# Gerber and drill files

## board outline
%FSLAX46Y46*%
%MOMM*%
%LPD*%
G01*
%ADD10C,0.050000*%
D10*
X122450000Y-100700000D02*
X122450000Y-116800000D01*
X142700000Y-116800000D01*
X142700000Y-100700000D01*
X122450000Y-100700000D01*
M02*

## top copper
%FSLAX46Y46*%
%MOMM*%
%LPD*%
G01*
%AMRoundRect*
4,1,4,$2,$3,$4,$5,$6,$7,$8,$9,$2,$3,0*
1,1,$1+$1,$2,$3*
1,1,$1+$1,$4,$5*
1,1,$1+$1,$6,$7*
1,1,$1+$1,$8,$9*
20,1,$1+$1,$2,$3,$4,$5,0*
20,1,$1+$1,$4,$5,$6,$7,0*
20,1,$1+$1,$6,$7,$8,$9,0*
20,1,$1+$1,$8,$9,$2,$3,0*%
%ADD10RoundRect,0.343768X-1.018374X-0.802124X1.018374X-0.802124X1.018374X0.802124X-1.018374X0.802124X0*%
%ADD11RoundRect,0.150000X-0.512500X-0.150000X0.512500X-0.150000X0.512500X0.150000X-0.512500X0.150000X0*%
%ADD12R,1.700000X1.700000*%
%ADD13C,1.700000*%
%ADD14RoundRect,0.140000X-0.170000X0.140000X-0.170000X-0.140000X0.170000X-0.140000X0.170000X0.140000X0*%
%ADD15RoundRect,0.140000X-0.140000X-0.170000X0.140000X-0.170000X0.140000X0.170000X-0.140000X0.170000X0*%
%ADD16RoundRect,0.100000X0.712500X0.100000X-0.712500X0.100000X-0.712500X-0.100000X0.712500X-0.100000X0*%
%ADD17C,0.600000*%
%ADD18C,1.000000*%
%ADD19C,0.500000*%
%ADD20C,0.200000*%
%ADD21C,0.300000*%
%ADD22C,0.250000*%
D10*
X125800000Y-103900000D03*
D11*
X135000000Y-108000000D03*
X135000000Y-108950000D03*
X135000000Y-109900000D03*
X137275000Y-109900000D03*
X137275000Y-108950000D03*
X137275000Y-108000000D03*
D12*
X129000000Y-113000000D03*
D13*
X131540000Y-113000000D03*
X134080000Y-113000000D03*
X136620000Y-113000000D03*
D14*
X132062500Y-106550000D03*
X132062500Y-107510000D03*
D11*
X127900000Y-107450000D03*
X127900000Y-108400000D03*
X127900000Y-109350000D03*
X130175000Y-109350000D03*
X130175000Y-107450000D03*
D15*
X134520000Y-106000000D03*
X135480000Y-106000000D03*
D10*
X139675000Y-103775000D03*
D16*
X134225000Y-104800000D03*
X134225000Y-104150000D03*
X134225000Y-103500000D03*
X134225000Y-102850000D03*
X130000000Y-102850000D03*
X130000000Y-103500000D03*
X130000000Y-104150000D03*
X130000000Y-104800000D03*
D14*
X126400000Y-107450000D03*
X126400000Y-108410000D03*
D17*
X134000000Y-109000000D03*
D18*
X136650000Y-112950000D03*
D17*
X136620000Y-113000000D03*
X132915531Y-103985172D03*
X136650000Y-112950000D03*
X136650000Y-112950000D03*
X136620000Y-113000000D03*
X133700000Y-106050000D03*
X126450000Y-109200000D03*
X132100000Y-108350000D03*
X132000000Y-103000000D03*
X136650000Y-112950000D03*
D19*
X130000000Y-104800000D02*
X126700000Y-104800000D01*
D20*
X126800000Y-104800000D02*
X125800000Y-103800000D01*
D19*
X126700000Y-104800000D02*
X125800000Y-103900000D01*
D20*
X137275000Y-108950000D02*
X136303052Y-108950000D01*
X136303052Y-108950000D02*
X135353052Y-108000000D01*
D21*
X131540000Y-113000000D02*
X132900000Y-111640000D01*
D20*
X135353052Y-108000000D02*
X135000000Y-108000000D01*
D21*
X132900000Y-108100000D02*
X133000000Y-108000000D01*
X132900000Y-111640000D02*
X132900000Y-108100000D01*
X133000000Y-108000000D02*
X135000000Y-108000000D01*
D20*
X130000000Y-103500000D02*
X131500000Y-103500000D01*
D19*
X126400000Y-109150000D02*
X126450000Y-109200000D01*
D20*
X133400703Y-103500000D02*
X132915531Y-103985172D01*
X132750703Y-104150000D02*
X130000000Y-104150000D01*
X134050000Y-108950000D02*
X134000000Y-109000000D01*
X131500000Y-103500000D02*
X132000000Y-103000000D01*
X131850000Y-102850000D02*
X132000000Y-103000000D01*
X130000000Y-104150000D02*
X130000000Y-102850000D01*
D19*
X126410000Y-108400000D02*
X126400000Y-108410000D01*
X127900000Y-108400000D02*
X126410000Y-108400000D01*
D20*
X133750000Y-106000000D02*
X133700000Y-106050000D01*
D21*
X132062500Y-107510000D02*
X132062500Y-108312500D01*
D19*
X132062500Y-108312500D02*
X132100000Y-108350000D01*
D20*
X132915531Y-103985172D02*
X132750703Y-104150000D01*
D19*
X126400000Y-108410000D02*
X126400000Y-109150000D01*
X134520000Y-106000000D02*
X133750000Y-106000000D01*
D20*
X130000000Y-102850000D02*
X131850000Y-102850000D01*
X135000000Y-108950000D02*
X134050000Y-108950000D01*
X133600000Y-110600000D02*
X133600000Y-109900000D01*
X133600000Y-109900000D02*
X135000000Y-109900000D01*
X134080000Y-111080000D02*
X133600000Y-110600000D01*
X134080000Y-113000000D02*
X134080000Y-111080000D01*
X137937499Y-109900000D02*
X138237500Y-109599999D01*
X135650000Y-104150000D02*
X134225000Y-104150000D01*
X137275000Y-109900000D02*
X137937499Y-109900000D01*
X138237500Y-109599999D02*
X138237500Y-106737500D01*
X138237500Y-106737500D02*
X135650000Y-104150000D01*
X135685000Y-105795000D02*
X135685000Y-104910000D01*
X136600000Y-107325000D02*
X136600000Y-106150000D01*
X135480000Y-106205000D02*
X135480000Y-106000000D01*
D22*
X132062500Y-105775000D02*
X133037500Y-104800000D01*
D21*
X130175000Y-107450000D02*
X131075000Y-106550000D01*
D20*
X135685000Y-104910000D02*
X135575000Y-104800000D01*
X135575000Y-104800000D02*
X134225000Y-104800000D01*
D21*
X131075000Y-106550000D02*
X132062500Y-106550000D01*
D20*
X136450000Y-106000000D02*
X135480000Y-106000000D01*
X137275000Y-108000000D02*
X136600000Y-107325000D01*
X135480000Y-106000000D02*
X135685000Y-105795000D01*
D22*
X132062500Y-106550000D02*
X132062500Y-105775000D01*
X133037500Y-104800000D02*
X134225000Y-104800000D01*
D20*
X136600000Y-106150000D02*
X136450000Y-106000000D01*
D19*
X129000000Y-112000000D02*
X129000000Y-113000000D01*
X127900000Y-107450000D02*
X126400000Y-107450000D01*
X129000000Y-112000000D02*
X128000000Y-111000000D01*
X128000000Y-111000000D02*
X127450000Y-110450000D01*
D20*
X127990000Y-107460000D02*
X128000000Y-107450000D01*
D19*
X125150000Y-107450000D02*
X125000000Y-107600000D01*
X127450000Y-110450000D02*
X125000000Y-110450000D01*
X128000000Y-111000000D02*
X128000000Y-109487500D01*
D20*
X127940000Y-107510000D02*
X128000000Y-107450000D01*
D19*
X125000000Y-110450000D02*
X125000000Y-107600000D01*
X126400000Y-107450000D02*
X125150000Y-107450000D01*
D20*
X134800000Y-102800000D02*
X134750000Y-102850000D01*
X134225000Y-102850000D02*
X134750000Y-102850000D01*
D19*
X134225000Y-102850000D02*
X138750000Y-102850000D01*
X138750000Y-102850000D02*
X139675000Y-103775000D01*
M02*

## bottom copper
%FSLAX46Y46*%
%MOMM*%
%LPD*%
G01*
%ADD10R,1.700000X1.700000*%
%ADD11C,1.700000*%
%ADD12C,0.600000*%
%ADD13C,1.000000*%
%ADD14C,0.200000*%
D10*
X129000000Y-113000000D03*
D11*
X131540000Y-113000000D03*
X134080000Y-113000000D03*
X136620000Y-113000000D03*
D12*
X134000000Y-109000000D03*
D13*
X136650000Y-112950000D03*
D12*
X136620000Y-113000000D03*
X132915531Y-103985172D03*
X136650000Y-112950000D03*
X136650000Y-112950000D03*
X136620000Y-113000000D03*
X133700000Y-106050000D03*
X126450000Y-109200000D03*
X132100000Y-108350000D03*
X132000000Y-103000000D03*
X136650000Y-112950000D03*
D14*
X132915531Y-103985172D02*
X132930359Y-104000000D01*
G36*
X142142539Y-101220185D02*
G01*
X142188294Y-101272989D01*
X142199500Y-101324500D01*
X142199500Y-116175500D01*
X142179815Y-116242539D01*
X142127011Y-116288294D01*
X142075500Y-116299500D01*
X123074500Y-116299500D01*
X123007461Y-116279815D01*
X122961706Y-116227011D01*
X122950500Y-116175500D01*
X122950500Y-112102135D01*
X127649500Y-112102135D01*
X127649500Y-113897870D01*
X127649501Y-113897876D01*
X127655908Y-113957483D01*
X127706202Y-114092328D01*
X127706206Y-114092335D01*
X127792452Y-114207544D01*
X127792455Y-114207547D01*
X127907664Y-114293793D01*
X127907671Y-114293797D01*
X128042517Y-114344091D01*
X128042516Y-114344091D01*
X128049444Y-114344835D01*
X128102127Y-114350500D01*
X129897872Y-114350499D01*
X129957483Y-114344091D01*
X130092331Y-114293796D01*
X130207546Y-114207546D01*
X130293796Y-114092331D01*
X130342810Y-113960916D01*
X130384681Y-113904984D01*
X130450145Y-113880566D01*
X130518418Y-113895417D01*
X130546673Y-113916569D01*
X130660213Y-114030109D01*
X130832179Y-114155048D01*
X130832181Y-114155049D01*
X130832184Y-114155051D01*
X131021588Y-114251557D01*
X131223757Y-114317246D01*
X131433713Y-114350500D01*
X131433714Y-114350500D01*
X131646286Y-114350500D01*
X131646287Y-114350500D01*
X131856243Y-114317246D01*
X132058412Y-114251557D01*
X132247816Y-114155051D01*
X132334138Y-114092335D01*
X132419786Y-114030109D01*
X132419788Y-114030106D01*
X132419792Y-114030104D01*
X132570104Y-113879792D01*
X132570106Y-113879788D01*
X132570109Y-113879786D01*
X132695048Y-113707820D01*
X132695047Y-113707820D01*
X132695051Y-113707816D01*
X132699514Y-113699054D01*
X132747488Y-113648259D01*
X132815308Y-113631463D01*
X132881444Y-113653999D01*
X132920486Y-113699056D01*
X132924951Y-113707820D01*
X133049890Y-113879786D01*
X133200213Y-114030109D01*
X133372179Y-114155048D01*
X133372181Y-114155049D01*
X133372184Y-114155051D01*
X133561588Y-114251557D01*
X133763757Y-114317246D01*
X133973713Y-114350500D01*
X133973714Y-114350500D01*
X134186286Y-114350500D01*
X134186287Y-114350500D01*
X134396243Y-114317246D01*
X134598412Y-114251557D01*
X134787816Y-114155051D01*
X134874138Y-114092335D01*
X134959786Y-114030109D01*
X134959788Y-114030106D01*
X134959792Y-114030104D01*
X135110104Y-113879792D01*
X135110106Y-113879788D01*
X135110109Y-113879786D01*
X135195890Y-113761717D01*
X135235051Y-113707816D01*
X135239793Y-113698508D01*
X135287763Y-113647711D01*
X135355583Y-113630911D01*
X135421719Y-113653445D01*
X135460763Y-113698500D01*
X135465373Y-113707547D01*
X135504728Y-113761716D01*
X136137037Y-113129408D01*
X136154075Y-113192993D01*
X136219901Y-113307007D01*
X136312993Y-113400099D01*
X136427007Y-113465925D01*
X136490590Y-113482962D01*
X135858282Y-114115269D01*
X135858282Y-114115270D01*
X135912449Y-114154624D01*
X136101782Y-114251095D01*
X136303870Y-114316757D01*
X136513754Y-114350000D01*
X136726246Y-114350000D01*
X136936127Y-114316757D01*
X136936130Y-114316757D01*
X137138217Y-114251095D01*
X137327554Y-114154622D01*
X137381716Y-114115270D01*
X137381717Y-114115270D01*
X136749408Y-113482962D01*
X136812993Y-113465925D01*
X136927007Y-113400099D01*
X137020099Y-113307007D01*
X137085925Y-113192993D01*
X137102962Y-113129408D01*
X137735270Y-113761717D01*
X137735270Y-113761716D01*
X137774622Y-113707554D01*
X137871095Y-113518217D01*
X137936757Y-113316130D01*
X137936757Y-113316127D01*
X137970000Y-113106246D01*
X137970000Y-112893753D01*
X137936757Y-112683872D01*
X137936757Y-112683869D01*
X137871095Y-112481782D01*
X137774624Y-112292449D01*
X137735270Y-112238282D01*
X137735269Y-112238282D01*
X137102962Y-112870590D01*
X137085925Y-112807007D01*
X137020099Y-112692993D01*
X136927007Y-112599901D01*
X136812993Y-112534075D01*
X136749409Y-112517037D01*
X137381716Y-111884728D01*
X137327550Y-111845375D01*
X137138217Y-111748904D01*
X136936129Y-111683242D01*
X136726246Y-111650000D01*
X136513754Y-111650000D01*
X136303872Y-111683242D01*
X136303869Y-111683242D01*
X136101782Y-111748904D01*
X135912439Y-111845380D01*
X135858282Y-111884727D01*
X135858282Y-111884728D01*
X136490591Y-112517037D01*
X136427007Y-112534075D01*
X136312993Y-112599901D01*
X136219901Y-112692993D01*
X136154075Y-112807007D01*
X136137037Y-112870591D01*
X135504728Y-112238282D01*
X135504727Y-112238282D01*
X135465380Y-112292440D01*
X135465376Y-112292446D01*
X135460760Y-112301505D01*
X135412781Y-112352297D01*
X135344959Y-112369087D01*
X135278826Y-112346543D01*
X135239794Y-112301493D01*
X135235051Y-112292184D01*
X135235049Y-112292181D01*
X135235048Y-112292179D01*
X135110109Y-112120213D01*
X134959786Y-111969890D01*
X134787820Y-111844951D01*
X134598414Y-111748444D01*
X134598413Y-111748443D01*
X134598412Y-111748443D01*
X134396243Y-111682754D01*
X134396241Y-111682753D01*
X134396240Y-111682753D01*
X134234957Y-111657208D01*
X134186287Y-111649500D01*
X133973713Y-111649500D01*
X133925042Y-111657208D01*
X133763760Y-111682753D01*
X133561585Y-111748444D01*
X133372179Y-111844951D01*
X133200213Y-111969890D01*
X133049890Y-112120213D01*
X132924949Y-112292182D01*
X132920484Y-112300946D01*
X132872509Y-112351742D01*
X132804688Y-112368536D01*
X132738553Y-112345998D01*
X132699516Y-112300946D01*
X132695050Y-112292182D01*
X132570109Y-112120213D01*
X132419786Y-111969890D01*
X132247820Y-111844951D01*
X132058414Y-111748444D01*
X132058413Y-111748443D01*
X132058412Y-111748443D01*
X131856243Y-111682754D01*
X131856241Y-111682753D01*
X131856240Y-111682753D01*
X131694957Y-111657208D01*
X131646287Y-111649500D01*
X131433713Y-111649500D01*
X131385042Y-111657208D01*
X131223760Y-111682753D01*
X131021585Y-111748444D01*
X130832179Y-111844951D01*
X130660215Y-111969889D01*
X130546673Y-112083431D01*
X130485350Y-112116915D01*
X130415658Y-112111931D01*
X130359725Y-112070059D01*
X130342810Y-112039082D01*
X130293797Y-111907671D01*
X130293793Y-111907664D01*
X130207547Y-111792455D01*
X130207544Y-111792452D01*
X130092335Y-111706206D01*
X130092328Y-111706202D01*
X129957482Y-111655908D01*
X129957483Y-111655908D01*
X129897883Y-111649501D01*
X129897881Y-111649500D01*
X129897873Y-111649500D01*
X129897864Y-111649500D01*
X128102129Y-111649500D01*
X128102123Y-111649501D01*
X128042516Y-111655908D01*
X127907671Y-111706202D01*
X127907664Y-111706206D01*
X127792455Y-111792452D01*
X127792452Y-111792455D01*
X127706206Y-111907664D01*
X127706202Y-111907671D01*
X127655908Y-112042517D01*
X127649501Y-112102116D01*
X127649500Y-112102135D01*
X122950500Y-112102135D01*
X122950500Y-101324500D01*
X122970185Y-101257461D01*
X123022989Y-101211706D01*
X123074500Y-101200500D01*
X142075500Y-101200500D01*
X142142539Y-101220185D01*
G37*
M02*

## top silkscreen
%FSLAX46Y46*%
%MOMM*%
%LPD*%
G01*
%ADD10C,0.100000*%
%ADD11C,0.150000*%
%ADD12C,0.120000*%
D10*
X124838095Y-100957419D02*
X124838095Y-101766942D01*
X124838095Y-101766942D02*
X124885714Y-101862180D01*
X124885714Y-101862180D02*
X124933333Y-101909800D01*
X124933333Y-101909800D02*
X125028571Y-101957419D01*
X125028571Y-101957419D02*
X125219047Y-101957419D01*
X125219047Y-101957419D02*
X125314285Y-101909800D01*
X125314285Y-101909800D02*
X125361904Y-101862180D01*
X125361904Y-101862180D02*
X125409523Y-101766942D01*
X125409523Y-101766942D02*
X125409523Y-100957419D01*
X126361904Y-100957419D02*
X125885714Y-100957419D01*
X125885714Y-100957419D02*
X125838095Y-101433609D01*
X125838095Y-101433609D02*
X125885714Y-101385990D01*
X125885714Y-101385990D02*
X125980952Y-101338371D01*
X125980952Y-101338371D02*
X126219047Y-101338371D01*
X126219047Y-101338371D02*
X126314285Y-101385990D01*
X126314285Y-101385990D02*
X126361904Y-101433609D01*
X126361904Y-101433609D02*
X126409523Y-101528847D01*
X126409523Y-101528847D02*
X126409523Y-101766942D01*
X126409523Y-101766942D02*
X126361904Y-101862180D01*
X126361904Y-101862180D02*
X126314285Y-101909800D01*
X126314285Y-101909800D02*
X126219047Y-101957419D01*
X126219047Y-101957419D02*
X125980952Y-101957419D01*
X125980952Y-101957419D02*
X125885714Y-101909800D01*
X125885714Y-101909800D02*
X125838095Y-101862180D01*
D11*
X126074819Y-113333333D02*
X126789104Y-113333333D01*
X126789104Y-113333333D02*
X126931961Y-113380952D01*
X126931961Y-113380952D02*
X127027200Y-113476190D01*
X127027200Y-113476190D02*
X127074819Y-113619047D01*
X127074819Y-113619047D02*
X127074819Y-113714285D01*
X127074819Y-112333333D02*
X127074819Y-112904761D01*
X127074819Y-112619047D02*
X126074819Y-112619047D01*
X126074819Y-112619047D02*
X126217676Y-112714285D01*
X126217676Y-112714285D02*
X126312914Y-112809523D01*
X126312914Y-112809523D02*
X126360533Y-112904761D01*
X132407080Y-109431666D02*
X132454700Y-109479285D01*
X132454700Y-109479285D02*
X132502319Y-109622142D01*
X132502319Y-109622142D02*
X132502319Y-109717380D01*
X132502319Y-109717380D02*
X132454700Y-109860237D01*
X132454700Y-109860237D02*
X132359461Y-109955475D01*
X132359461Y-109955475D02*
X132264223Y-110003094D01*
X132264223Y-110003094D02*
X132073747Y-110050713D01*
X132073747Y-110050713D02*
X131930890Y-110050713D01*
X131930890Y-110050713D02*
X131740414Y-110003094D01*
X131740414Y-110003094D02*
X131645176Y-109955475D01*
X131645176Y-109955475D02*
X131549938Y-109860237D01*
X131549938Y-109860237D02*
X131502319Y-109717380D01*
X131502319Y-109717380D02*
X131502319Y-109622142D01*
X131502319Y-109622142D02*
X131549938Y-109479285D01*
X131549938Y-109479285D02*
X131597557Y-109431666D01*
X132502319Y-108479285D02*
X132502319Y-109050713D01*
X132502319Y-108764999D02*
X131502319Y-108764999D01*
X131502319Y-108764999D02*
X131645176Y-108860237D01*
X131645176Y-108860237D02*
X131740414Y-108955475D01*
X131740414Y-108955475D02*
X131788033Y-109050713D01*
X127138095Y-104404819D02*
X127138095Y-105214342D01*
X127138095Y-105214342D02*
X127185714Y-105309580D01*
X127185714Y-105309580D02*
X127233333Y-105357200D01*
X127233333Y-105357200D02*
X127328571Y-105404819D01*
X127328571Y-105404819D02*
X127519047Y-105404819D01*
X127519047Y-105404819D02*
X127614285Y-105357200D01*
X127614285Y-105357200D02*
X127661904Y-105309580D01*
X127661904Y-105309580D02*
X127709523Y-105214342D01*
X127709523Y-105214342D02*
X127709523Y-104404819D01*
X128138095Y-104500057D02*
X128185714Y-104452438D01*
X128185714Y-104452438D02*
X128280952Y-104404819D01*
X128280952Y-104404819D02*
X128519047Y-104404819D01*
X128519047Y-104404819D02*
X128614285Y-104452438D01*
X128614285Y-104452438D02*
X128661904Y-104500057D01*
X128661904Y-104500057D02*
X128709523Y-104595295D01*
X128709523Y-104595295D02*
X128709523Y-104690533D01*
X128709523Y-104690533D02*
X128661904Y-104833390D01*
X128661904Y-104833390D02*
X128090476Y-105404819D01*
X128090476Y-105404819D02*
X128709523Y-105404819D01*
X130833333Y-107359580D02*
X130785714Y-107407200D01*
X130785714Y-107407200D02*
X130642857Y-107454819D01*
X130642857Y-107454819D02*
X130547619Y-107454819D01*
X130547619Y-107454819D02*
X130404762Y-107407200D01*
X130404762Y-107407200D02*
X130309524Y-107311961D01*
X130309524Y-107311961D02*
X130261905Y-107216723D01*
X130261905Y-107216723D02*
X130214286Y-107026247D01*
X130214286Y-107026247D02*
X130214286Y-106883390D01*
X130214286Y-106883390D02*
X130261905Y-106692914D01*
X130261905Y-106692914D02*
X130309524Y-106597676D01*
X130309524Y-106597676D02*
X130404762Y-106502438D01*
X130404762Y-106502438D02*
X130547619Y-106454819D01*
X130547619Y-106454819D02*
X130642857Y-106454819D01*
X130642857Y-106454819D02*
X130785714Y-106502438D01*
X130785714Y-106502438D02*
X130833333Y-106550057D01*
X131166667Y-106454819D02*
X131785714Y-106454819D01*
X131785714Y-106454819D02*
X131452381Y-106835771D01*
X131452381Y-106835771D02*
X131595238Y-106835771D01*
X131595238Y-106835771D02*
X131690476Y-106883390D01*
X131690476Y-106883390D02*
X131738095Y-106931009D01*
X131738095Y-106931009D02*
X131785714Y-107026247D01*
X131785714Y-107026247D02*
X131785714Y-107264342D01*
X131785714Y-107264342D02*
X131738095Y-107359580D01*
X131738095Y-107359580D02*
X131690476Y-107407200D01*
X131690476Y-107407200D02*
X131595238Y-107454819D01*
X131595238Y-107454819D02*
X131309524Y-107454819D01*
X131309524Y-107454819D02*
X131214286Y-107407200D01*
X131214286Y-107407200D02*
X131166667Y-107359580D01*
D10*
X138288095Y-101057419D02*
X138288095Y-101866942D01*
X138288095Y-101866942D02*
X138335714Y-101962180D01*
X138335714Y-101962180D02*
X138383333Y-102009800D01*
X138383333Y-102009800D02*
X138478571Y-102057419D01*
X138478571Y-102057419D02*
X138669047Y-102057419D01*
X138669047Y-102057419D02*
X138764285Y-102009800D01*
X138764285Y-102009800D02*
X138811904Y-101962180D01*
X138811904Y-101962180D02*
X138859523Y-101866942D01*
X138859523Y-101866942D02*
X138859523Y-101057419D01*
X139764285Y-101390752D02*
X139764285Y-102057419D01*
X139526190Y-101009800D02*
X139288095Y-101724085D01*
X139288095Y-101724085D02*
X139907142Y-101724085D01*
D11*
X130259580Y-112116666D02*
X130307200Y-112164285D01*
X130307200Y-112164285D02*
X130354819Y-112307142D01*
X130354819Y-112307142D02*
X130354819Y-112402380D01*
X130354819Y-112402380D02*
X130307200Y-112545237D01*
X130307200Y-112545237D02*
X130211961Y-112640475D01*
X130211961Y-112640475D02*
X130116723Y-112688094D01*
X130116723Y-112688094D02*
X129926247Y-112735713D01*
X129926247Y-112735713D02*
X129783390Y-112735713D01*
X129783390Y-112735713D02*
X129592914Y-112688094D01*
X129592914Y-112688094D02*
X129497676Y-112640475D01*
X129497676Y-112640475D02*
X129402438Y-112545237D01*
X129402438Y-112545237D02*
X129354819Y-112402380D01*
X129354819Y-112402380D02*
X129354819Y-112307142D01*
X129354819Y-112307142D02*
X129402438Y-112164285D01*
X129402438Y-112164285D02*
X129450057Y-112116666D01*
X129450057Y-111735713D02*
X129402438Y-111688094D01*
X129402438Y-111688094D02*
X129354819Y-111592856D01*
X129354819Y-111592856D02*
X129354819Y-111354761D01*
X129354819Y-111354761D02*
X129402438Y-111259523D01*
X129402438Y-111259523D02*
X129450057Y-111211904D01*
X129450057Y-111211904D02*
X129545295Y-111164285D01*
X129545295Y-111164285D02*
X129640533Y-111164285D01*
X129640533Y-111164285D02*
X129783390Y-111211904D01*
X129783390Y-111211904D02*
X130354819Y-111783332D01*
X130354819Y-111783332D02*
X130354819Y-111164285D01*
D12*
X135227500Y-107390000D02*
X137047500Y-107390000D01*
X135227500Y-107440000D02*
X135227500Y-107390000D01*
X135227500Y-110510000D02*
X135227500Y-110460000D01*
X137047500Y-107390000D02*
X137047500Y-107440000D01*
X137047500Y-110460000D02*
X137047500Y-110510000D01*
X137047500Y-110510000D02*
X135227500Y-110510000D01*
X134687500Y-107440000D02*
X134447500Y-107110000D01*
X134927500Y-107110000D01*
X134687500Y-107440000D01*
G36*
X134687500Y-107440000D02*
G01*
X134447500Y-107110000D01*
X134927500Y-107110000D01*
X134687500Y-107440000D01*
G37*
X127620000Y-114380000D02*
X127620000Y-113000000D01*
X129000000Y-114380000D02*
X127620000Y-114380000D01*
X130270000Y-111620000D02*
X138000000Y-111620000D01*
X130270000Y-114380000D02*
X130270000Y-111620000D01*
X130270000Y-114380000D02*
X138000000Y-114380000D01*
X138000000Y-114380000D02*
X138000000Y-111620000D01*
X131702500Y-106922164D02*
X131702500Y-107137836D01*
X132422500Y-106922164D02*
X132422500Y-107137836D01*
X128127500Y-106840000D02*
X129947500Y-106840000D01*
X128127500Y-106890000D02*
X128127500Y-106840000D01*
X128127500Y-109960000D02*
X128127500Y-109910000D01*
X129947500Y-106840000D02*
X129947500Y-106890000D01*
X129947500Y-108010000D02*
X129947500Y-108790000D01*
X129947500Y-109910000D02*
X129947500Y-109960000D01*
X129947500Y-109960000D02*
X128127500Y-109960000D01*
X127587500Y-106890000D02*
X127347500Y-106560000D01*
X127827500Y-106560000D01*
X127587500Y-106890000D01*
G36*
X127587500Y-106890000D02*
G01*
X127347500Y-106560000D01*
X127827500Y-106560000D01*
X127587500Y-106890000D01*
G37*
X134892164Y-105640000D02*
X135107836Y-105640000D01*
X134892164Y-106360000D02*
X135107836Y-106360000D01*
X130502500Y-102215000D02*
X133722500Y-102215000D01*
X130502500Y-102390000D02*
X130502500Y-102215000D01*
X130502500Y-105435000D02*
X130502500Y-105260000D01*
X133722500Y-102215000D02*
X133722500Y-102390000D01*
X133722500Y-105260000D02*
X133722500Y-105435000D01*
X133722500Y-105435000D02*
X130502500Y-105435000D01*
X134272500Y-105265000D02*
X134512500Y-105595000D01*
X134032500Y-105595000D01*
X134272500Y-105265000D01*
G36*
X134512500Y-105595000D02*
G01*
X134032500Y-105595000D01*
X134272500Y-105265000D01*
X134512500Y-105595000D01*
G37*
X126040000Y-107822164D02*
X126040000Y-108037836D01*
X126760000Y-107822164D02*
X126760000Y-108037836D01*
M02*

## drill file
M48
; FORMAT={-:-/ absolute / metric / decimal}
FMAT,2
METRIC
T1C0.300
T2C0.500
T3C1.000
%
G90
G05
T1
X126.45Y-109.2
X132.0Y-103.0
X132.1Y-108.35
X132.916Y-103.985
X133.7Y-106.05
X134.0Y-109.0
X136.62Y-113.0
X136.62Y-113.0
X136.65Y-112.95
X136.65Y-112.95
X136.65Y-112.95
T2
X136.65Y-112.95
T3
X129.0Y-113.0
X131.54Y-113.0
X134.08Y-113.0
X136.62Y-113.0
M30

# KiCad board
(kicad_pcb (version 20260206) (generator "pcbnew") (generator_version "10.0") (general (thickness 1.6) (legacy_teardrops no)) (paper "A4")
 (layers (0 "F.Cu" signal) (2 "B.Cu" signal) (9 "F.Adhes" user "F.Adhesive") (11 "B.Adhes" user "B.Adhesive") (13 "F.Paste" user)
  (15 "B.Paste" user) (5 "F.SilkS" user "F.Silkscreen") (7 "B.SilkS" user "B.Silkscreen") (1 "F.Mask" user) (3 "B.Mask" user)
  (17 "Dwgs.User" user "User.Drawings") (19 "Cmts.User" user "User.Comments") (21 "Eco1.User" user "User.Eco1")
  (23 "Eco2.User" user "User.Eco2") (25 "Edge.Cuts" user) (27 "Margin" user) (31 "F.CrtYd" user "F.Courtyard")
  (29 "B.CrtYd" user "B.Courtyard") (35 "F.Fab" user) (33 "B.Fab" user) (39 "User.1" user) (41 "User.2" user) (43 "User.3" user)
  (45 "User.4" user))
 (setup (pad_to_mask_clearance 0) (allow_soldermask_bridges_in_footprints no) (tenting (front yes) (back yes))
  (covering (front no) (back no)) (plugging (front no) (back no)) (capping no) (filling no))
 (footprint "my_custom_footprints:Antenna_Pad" (layer "F.Cu") (at 125.8 103.9)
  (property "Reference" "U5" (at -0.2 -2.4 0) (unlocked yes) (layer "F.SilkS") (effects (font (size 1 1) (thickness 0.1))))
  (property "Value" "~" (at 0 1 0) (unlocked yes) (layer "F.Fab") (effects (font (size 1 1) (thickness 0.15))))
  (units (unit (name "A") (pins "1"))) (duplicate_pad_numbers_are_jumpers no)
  (pad "1" smd roundrect (at 0 0) (size 2.724284 2.291785) (layers "F.Cu" "F.Mask" "F.Paste") (roundrect_rratio 0.15) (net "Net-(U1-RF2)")))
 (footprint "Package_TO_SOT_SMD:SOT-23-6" (layer "F.Cu") (at 136.1375 108.95)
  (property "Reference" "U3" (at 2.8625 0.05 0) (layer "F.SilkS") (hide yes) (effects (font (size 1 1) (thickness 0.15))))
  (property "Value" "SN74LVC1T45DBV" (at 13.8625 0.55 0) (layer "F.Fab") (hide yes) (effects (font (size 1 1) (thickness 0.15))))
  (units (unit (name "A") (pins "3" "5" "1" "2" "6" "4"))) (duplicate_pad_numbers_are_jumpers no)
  (fp_line (start -0.91 -1.56) (end 0.91 -1.56) (stroke (width 0.12) (type solid)) (layer "F.SilkS"))
  (fp_line (start -0.91 -1.51) (end -0.91 -1.56) (stroke (width 0.12) (type solid)) (layer "F.SilkS"))
  (fp_line (start -0.91 1.56) (end -0.91 1.51) (stroke (width 0.12) (type solid)) (layer "F.SilkS"))
  (fp_line (start 0.91 -1.56) (end 0.91 -1.51) (stroke (width 0.12) (type solid)) (layer "F.SilkS"))
  (fp_line (start 0.91 1.51) (end 0.91 1.56) (stroke (width 0.12) (type solid)) (layer "F.SilkS"))
  (fp_line (start 0.91 1.56) (end -0.91 1.56) (stroke (width 0.12) (type solid)) (layer "F.SilkS"))
  (fp_poly (pts (xy -1.45 -1.51) (xy -1.69 -1.84) (xy -1.21 -1.84)) (stroke (width 0.12) (type solid)) (fill yes) (layer "F.SilkS"))
  (pad "1" smd roundrect (at -1.1375 -0.95) (size 1.325 0.6) (layers "F.Cu" "F.Mask" "F.Paste") (roundrect_rratio 0.25) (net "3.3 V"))
  (pad "2" smd roundrect (at -1.1375 0) (size 1.325 0.6) (layers "F.Cu" "F.Mask" "F.Paste") (roundrect_rratio 0.25) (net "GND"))
  (pad "3" smd roundrect (at -1.1375 0.95) (size 1.325 0.6) (layers "F.Cu" "F.Mask" "F.Paste") (roundrect_rratio 0.25)
   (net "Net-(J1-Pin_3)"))
  (pad "4" smd roundrect (at 1.1375 0.95) (size 1.325 0.6) (layers "F.Cu" "F.Mask" "F.Paste") (roundrect_rratio 0.25) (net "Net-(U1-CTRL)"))
  (pad "5" smd roundrect (at 1.1375 0) (size 1.325 0.6) (layers "F.Cu" "F.Mask" "F.Paste") (roundrect_rratio 0.25) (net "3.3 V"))
  (pad "6" smd roundrect (at 1.1375 -0.95) (size 1.325 0.6) (layers "F.Cu" "F.Mask" "F.Paste") (roundrect_rratio 0.25) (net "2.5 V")))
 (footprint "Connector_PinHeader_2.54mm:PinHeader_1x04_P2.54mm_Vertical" (layer "F.Cu") (at 129 113 90)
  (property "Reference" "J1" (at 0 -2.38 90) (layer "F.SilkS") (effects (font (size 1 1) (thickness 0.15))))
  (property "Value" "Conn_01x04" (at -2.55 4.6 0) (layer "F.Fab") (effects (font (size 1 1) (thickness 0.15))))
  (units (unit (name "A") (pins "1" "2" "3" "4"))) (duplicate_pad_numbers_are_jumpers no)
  (fp_line (start -1.38 -1.38) (end 0 -1.38) (stroke (width 0.12) (type solid)) (layer "F.SilkS"))
  (fp_line (start -1.38 0) (end -1.38 -1.38) (stroke (width 0.12) (type solid)) (layer "F.SilkS"))
  (fp_line (start 1.38 1.27) (end 1.38 9) (stroke (width 0.12) (type solid)) (layer "F.SilkS"))
  (fp_line (start -1.38 1.27) (end 1.38 1.27) (stroke (width 0.12) (type solid)) (layer "F.SilkS"))
  (fp_line (start -1.38 1.27) (end -1.38 9) (stroke (width 0.12) (type solid)) (layer "F.SilkS"))
  (fp_line (start -1.38 9) (end 1.38 9) (stroke (width 0.12) (type solid)) (layer "F.SilkS"))
  (pad "1" thru_hole rect (at 0 0 90) (size 1.7 1.7) (drill 1) (layers "*.Cu" "*.Mask") (remove_unused_layers no) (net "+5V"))
  (pad "2" thru_hole circle (at 0 2.54 90) (size 1.7 1.7) (drill 1) (layers "*.Cu" "*.Mask") (remove_unused_layers no) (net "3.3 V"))
  (pad "3" thru_hole circle (at 0 5.08 90) (size 1.7 1.7) (drill 1) (layers "*.Cu" "*.Mask") (remove_unused_layers no)
   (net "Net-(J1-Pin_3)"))
  (pad "4" thru_hole circle (at 0 7.62 90) (size 1.7 1.7) (drill 1) (layers "*.Cu" "*.Mask") (remove_unused_layers no) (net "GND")))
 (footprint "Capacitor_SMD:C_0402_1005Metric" (layer "F.Cu") (at 132.0625 107.03 -90)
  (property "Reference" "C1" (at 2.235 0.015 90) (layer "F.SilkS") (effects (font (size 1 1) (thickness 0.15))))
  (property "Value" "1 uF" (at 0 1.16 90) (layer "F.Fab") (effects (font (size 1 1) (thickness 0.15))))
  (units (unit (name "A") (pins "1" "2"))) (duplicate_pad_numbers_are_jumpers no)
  (fp_line (start -0.107836 0.36) (end 0.107836 0.36) (stroke (width 0.12) (type solid)) (layer "F.SilkS"))
  (fp_line (start -0.107836 -0.36) (end 0.107836 -0.36) (stroke (width 0.12) (type solid)) (layer "F.SilkS"))
  (pad "1" smd roundrect (at -0.48 0 270) (size 0.56 0.62) (layers "F.Cu" "F.Mask" "F.Paste") (roundrect_rratio 0.25) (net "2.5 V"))
  (pad "2" smd roundrect (at 0.48 0 270) (size 0.56 0.62) (layers "F.Cu" "F.Mask" "F.Paste") (roundrect_rratio 0.25) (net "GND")))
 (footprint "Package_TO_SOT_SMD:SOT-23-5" (layer "F.Cu") (at 129.0375 108.4)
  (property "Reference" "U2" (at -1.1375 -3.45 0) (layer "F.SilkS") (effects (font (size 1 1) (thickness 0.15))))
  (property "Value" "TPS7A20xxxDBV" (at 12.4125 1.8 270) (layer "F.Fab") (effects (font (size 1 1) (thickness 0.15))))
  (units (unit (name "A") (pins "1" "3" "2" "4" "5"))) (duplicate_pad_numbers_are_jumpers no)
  (fp_line (start -0.91 -1.56) (end 0.91 -1.56) (stroke (width 0.12) (type solid)) (layer "F.SilkS"))
  (fp_line (start -0.91 -1.51) (end -0.91 -1.56) (stroke (width 0.12) (type solid)) (layer "F.SilkS"))
  (fp_line (start -0.91 1.56) (end -0.91 1.51) (stroke (width 0.12) (type solid)) (layer "F.SilkS"))
  (fp_line (start 0.91 -1.56) (end 0.91 -1.51) (stroke (width 0.12) (type solid)) (layer "F.SilkS"))
  (fp_line (start 0.91 -0.39) (end 0.91 0.39) (stroke (width 0.12) (type solid)) (layer "F.SilkS"))
  (fp_line (start 0.91 1.51) (end 0.91 1.56) (stroke (width 0.12) (type solid)) (layer "F.SilkS"))
  (fp_line (start 0.91 1.56) (end -0.91 1.56) (stroke (width 0.12) (type solid)) (layer "F.SilkS"))
  (fp_poly (pts (xy -1.45 -1.51) (xy -1.69 -1.84) (xy -1.21 -1.84)) (stroke (width 0.12) (type solid)) (fill yes) (layer "F.SilkS"))
  (pad "1" smd roundrect (at -1.1375 -0.95) (size 1.325 0.6) (layers "F.Cu" "F.Mask" "F.Paste") (roundrect_rratio 0.25) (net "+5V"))
  (pad "2" smd roundrect (at -1.1375 0) (size 1.325 0.6) (layers "F.Cu" "F.Mask" "F.Paste") (roundrect_rratio 0.25) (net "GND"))
  (pad "3" smd roundrect (at -1.1375 0.95) (size 1.325 0.6) (layers "F.Cu" "F.Mask" "F.Paste") (roundrect_rratio 0.25) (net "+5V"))
  (pad "4" smd roundrect (at 1.1375 0.95) (size 1.325 0.6) (layers "F.Cu" "F.Mask" "F.Paste") (roundrect_rratio 0.25)
   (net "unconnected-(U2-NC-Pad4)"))
  (pad "5" smd roundrect (at 1.1375 -0.95) (size 1.325 0.6) (layers "F.Cu" "F.Mask" "F.Paste") (roundrect_rratio 0.25) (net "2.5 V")))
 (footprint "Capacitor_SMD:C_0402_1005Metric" (layer "F.Cu") (at 135 106)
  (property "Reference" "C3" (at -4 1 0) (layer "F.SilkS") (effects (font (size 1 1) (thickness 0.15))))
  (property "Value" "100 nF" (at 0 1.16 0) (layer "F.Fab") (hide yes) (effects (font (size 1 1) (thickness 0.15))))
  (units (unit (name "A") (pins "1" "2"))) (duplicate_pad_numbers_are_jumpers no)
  (fp_line (start -0.107836 -0.36) (end 0.107836 -0.36) (stroke (width 0.12) (type solid)) (layer "F.SilkS"))
  (fp_line (start -0.107836 0.36) (end 0.107836 0.36) (stroke (width 0.12) (type solid)) (layer "F.SilkS"))
  (pad "1" smd roundrect (at -0.48 0) (size 0.56 0.62) (layers "F.Cu" "F.Mask" "F.Paste") (roundrect_rratio 0.25) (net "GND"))
  (pad "2" smd roundrect (at 0.48 0) (size 0.56 0.62) (layers "F.Cu" "F.Mask" "F.Paste") (roundrect_rratio 0.25) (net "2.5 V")))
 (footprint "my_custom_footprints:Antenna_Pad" (layer "F.Cu") (at 139.675 103.775)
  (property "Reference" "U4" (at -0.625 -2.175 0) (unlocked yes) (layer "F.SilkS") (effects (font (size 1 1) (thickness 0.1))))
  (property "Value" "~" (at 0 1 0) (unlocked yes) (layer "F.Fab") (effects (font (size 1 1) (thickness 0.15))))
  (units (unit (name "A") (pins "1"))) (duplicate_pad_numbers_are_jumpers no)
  (pad "1" smd roundrect (at 0 0) (size 2.724284 2.291785) (layers "F.Cu" "F.Mask" "F.Paste") (roundrect_rratio 0.15) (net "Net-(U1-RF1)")))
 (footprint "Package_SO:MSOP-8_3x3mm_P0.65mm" (layer "F.Cu") (at 132.1125 103.825 180)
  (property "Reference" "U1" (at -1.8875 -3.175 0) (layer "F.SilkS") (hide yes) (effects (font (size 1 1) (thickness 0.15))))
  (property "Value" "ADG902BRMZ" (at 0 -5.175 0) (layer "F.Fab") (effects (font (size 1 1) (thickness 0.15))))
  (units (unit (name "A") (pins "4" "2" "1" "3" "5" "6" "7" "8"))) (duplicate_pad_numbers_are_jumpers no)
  (fp_line (start 1.61 1.61) (end -1.61 1.61) (stroke (width 0.12) (type solid)) (layer "F.SilkS"))
  (fp_line (start 1.61 1.435) (end 1.61 1.61) (stroke (width 0.12) (type solid)) (layer "F.SilkS"))
  (fp_line (start 1.61 -1.61) (end 1.61 -1.435) (stroke (width 0.12) (type solid)) (layer "F.SilkS"))
  (fp_line (start -1.61 1.61) (end -1.61 1.435) (stroke (width 0.12) (type solid)) (layer "F.SilkS"))
  (fp_line (start -1.61 -1.435) (end -1.61 -1.61) (stroke (width 0.12) (type solid)) (layer "F.SilkS"))
  (fp_line (start -1.61 -1.61) (end 1.61 -1.61) (stroke (width 0.12) (type solid)) (layer "F.SilkS"))
  (fp_poly (pts (xy -2.16 -1.44) (xy -2.4 -1.77) (xy -1.92 -1.77)) (stroke (width 0.12) (type solid)) (fill yes) (layer "F.SilkS"))
  (pad "1" smd roundrect (at -2.1125 -0.975 180) (size 1.625 0.4) (layers "F.Cu" "F.Mask" "F.Paste") (roundrect_rratio 0.25) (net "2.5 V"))
  (pad "2" smd roundrect (at -2.1125 -0.325 180) (size 1.625 0.4) (layers "F.Cu" "F.Mask" "F.Paste") (roundrect_rratio 0.25)
   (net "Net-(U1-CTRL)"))
  (pad "3" smd roundrect (at -2.1125 0.325 180) (size 1.625 0.4) (layers "F.Cu" "F.Mask" "F.Paste") (roundrect_rratio 0.25) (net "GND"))
  (pad "4" smd roundrect (at -2.1125 0.975 180) (size 1.625 0.4) (layers "F.Cu" "F.Mask" "F.Paste") (roundrect_rratio 0.25)
   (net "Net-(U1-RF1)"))
  (pad "5" smd roundrect (at 2.1125 0.975 180) (size 1.625 0.4) (layers "F.Cu" "F.Mask" "F.Paste") (roundrect_rratio 0.25) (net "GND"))
  (pad "6" smd roundrect (at 2.1125 0.325 180) (size 1.625 0.4) (layers "F.Cu" "F.Mask" "F.Paste") (roundrect_rratio 0.25) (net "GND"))
  (pad "7" smd roundrect (at 2.1125 -0.325 180) (size 1.625 0.4) (layers "F.Cu" "F.Mask" "F.Paste") (roundrect_rratio 0.25) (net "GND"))
  (pad "8" smd roundrect (at 2.1125 -0.975 180) (size 1.625 0.4) (layers "F.Cu" "F.Mask" "F.Paste") (roundrect_rratio 0.25)
   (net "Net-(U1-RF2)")))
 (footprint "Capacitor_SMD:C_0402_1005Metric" (layer "F.Cu") (at 126.4 107.93 -90)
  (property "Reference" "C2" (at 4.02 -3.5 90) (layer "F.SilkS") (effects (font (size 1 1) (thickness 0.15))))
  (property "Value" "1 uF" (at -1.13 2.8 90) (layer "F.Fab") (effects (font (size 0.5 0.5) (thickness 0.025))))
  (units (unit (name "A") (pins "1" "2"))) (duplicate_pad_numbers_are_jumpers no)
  (fp_line (start -0.107836 0.36) (end 0.107836 0.36) (stroke (width 0.12) (type solid)) (layer "F.SilkS"))
  (fp_line (start -0.107836 -0.36) (end 0.107836 -0.36) (stroke (width 0.12) (type solid)) (layer "F.SilkS"))
  (pad "1" smd roundrect (at -0.48 0 270) (size 0.56 0.62) (layers "F.Cu" "F.Mask" "F.Paste") (roundrect_rratio 0.25) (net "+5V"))
  (pad "2" smd roundrect (at 0.48 0 270) (size 0.56 0.62) (layers "F.Cu" "F.Mask" "F.Paste") (roundrect_rratio 0.25) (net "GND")))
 (gr_poly
  (pts (xy 122.45 100.7) (xy 122.45 116.8) (xy 142.7 116.8) (xy 142.7 100.7)) (stroke (width 0.05) (type solid)) (fill no)
  (layer "Edge.Cuts"))
 (segment (start 130 104.8) (end 126.7 104.8) (width 0.5) (layer "F.Cu") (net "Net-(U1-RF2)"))
 (segment (start 126.8 104.8) (end 125.8 103.8) (width 0.2) (layer "F.Cu") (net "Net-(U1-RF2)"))
 (segment (start 126.7 104.8) (end 125.8 103.9) (width 0.5) (layer "F.Cu") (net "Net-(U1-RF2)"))
 (segment (start 137.275 108.95) (end 136.303052 108.95) (width 0.2) (layer "F.Cu") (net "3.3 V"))
 (segment (start 136.303052 108.95) (end 135.353052 108) (width 0.2) (layer "F.Cu") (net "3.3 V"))
 (segment (start 131.54 113) (end 132.9 111.64) (width 0.3) (layer "F.Cu") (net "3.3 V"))
 (segment (start 135.353052 108) (end 135 108) (width 0.2) (layer "F.Cu") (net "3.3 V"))
 (segment (start 132.9 108.1) (end 133 108) (width 0.3) (layer "F.Cu") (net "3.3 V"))
 (segment (start 132.9 111.64) (end 132.9 108.1) (width 0.3) (layer "F.Cu") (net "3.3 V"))
 (segment (start 133 108) (end 135 108) (width 0.3) (layer "F.Cu") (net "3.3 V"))
 (segment (start 130 103.5) (end 131.5 103.5) (width 0.2) (layer "F.Cu") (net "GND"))
 (segment (start 126.4 109.15) (end 126.45 109.2) (width 0.5) (layer "F.Cu") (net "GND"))
 (segment (start 133.400703 103.5) (end 132.915531 103.985172) (width 0.2) (layer "F.Cu") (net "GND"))
 (segment (start 132.750703 104.15) (end 130 104.15) (width 0.2) (layer "F.Cu") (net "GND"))
 (segment (start 134.05 108.95) (end 134 109) (width 0.2) (layer "F.Cu") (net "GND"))
 (segment (start 131.5 103.5) (end 132 103) (width 0.2) (layer "F.Cu") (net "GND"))
 (segment (start 131.85 102.85) (end 132 103) (width 0.2) (layer "F.Cu") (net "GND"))
 (segment (start 130 104.15) (end 130 102.85) (width 0.2) (layer "F.Cu") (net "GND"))
 (segment (start 126.41 108.4) (end 126.4 108.41) (width 0.5) (layer "F.Cu") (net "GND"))
 (segment (start 127.9 108.4) (end 126.41 108.4) (width 0.5) (layer "F.Cu") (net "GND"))
 (segment (start 133.75 106) (end 133.7 106.05) (width 0.2) (layer "F.Cu") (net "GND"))
 (segment (start 132.0625 107.51) (end 132.0625 108.3125) (width 0.3) (layer "F.Cu") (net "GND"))
 (segment (start 132.0625 108.3125) (end 132.1 108.35) (width 0.5) (layer "F.Cu") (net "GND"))
 (segment (start 132.915531 103.985172) (end 132.750703 104.15) (width 0.2) (layer "F.Cu") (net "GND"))
 (segment (start 126.4 108.41) (end 126.4 109.15) (width 0.5) (layer "F.Cu") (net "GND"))
 (segment (start 134.52 106) (end 133.75 106) (width 0.5) (layer "F.Cu") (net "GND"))
 (segment (start 130 102.85) (end 131.85 102.85) (width 0.2) (layer "F.Cu") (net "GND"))
 (segment (start 135 108.95) (end 134.05 108.95) (width 0.2) (layer "F.Cu") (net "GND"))
 (via (at 134 109) (size 0.6) (drill 0.3) (layers "F.Cu" "B.Cu") (free yes) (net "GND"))
 (via (at 136.65 112.95) (size 1) (drill 0.5) (layers "F.Cu" "B.Cu") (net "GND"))
 (via (at 136.62 113) (size 0.6) (drill 0.3) (layers "F.Cu" "B.Cu") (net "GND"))
 (via (at 132.915531 103.985172) (size 0.6) (drill 0.3) (layers "F.Cu" "B.Cu") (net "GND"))
 (via (at 136.65 112.95) (size 0.6) (drill 0.3) (layers "F.Cu" "B.Cu") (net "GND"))
 (via (at 136.65 112.95) (size 0.6) (drill 0.3) (layers "F.Cu" "B.Cu") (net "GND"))
 (via (at 136.62 113) (size 0.6) (drill 0.3) (layers "F.Cu" "B.Cu") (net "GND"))
 (via (at 133.7 106.05) (size 0.6) (drill 0.3) (layers "F.Cu" "B.Cu") (free yes) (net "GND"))
 (via (at 126.45 109.2) (size 0.6) (drill 0.3) (layers "F.Cu" "B.Cu") (free yes) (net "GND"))
 (via (at 132.1 108.35) (size 0.6) (drill 0.3) (layers "F.Cu" "B.Cu") (free yes) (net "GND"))
 (via (at 132 103) (size 0.6) (drill 0.3) (layers "F.Cu" "B.Cu") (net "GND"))
 (via (at 136.65 112.95) (size 0.6) (drill 0.3) (layers "F.Cu" "B.Cu") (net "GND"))
 (segment (start 132.915531 103.985172) (end 132.930359 104) (width 0.2) (layer "B.Cu") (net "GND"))
 (segment (start 133.6 110.6) (end 133.6 109.9) (width 0.2) (layer "F.Cu") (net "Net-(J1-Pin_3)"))
 (segment (start 133.6 109.9) (end 135 109.9) (width 0.2) (layer "F.Cu") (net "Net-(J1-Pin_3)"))
 (segment (start 134.08 111.08) (end 133.6 110.6) (width 0.2) (layer "F.Cu") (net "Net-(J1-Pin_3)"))
 (segment (start 134.08 113) (end 134.08 111.08) (width 0.2) (layer "F.Cu") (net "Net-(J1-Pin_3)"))
 (segment (start 137.937499 109.9) (end 138.2375 109.599999) (width 0.2) (layer "F.Cu") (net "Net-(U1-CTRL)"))
 (segment (start 135.65 104.15) (end 134.225 104.15) (width 0.2) (layer "F.Cu") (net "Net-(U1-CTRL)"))
 (segment (start 137.275 109.9) (end 137.937499 109.9) (width 0.2) (layer "F.Cu") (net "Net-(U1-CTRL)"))
 (segment (start 138.2375 109.599999) (end 138.2375 106.7375) (width 0.2) (layer "F.Cu") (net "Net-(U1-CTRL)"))
 (segment (start 138.2375 106.7375) (end 135.65 104.15) (width 0.2) (layer "F.Cu") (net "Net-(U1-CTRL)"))
 (segment (start 135.685 105.795) (end 135.685 104.91) (width 0.2) (layer "F.Cu") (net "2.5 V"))
 (segment (start 136.6 107.325) (end 136.6 106.15) (width 0.2) (layer "F.Cu") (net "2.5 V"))
 (segment (start 135.48 106.205) (end 135.48 106) (width 0.2) (layer "F.Cu") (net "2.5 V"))
 (segment (start 132.0625 105.775) (end 133.0375 104.8) (width 0.25) (layer "F.Cu") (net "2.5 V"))
 (segment (start 130.175 107.45) (end 131.075 106.55) (width 0.3) (layer "F.Cu") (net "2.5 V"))
 (segment (start 135.685 104.91) (end 135.575 104.8) (width 0.2) (layer "F.Cu") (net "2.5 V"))
 (segment (start 135.575 104.8) (end 134.225 104.8) (width 0.2) (layer "F.Cu") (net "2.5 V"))
 (segment (start 131.075 106.55) (end 132.0625 106.55) (width 0.3) (layer "F.Cu") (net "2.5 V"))
 (segment (start 136.45 106) (end 135.48 106) (width 0.2) (layer "F.Cu") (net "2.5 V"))
 (segment (start 137.275 108) (end 136.6 107.325) (width 0.2) (layer "F.Cu") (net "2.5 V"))
 (segment (start 135.48 106) (end 135.685 105.795) (width 0.2) (layer "F.Cu") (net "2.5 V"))
 (segment (start 132.0625 106.55) (end 132.0625 105.775) (width 0.25) (layer "F.Cu") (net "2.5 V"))
 (segment (start 133.0375 104.8) (end 134.225 104.8) (width 0.25) (layer "F.Cu") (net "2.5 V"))
 (segment (start 136.6 106.15) (end 136.45 106) (width 0.2) (layer "F.Cu") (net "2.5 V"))
 (segment (start 129 112) (end 129 113) (width 0.5) (layer "F.Cu") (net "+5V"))
 (segment (start 127.9 107.45) (end 126.4 107.45) (width 0.5) (layer "F.Cu") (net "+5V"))
 (segment (start 129 112) (end 128 111) (width 0.5) (layer "F.Cu") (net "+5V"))
 (segment (start 128 111) (end 127.45 110.45) (width 0.5) (layer "F.Cu") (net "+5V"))
 (segment (start 127.99 107.46) (end 128 107.45) (width 0.2) (layer "F.Cu") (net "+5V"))
 (segment (start 125.15 107.45) (end 125 107.6) (width 0.5) (layer "F.Cu") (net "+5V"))
 (segment (start 127.45 110.45) (end 125 110.45) (width 0.5) (layer "F.Cu") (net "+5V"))
 (segment (start 128 111) (end 128 109.4875) (width 0.5) (layer "F.Cu") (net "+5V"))
 (segment (start 127.94 107.51) (end 128 107.45) (width 0.2) (layer "F.Cu") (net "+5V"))
 (segment (start 125 110.45) (end 125 107.6) (width 0.5) (layer "F.Cu") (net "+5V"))
 (segment (start 126.4 107.45) (end 125.15 107.45) (width 0.5) (layer "F.Cu") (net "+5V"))
 (segment (start 134.8 102.8) (end 134.75 102.85) (width 0.2) (layer "F.Cu") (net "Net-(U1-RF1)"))
 (segment (start 134.225 102.85) (end 134.75 102.85) (width 0.2) (layer "F.Cu") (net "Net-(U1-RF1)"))
 (segment (start 134.225 102.85) (end 138.75 102.85) (width 0.5) (layer "F.Cu") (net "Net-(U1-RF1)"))
 (segment (start 138.75 102.85) (end 139.675 103.775) (width 0.5) (layer "F.Cu") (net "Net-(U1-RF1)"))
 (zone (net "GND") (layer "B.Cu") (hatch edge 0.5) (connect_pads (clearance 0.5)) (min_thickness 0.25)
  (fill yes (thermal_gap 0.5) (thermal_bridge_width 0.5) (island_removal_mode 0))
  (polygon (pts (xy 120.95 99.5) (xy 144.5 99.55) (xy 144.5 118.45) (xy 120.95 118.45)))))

